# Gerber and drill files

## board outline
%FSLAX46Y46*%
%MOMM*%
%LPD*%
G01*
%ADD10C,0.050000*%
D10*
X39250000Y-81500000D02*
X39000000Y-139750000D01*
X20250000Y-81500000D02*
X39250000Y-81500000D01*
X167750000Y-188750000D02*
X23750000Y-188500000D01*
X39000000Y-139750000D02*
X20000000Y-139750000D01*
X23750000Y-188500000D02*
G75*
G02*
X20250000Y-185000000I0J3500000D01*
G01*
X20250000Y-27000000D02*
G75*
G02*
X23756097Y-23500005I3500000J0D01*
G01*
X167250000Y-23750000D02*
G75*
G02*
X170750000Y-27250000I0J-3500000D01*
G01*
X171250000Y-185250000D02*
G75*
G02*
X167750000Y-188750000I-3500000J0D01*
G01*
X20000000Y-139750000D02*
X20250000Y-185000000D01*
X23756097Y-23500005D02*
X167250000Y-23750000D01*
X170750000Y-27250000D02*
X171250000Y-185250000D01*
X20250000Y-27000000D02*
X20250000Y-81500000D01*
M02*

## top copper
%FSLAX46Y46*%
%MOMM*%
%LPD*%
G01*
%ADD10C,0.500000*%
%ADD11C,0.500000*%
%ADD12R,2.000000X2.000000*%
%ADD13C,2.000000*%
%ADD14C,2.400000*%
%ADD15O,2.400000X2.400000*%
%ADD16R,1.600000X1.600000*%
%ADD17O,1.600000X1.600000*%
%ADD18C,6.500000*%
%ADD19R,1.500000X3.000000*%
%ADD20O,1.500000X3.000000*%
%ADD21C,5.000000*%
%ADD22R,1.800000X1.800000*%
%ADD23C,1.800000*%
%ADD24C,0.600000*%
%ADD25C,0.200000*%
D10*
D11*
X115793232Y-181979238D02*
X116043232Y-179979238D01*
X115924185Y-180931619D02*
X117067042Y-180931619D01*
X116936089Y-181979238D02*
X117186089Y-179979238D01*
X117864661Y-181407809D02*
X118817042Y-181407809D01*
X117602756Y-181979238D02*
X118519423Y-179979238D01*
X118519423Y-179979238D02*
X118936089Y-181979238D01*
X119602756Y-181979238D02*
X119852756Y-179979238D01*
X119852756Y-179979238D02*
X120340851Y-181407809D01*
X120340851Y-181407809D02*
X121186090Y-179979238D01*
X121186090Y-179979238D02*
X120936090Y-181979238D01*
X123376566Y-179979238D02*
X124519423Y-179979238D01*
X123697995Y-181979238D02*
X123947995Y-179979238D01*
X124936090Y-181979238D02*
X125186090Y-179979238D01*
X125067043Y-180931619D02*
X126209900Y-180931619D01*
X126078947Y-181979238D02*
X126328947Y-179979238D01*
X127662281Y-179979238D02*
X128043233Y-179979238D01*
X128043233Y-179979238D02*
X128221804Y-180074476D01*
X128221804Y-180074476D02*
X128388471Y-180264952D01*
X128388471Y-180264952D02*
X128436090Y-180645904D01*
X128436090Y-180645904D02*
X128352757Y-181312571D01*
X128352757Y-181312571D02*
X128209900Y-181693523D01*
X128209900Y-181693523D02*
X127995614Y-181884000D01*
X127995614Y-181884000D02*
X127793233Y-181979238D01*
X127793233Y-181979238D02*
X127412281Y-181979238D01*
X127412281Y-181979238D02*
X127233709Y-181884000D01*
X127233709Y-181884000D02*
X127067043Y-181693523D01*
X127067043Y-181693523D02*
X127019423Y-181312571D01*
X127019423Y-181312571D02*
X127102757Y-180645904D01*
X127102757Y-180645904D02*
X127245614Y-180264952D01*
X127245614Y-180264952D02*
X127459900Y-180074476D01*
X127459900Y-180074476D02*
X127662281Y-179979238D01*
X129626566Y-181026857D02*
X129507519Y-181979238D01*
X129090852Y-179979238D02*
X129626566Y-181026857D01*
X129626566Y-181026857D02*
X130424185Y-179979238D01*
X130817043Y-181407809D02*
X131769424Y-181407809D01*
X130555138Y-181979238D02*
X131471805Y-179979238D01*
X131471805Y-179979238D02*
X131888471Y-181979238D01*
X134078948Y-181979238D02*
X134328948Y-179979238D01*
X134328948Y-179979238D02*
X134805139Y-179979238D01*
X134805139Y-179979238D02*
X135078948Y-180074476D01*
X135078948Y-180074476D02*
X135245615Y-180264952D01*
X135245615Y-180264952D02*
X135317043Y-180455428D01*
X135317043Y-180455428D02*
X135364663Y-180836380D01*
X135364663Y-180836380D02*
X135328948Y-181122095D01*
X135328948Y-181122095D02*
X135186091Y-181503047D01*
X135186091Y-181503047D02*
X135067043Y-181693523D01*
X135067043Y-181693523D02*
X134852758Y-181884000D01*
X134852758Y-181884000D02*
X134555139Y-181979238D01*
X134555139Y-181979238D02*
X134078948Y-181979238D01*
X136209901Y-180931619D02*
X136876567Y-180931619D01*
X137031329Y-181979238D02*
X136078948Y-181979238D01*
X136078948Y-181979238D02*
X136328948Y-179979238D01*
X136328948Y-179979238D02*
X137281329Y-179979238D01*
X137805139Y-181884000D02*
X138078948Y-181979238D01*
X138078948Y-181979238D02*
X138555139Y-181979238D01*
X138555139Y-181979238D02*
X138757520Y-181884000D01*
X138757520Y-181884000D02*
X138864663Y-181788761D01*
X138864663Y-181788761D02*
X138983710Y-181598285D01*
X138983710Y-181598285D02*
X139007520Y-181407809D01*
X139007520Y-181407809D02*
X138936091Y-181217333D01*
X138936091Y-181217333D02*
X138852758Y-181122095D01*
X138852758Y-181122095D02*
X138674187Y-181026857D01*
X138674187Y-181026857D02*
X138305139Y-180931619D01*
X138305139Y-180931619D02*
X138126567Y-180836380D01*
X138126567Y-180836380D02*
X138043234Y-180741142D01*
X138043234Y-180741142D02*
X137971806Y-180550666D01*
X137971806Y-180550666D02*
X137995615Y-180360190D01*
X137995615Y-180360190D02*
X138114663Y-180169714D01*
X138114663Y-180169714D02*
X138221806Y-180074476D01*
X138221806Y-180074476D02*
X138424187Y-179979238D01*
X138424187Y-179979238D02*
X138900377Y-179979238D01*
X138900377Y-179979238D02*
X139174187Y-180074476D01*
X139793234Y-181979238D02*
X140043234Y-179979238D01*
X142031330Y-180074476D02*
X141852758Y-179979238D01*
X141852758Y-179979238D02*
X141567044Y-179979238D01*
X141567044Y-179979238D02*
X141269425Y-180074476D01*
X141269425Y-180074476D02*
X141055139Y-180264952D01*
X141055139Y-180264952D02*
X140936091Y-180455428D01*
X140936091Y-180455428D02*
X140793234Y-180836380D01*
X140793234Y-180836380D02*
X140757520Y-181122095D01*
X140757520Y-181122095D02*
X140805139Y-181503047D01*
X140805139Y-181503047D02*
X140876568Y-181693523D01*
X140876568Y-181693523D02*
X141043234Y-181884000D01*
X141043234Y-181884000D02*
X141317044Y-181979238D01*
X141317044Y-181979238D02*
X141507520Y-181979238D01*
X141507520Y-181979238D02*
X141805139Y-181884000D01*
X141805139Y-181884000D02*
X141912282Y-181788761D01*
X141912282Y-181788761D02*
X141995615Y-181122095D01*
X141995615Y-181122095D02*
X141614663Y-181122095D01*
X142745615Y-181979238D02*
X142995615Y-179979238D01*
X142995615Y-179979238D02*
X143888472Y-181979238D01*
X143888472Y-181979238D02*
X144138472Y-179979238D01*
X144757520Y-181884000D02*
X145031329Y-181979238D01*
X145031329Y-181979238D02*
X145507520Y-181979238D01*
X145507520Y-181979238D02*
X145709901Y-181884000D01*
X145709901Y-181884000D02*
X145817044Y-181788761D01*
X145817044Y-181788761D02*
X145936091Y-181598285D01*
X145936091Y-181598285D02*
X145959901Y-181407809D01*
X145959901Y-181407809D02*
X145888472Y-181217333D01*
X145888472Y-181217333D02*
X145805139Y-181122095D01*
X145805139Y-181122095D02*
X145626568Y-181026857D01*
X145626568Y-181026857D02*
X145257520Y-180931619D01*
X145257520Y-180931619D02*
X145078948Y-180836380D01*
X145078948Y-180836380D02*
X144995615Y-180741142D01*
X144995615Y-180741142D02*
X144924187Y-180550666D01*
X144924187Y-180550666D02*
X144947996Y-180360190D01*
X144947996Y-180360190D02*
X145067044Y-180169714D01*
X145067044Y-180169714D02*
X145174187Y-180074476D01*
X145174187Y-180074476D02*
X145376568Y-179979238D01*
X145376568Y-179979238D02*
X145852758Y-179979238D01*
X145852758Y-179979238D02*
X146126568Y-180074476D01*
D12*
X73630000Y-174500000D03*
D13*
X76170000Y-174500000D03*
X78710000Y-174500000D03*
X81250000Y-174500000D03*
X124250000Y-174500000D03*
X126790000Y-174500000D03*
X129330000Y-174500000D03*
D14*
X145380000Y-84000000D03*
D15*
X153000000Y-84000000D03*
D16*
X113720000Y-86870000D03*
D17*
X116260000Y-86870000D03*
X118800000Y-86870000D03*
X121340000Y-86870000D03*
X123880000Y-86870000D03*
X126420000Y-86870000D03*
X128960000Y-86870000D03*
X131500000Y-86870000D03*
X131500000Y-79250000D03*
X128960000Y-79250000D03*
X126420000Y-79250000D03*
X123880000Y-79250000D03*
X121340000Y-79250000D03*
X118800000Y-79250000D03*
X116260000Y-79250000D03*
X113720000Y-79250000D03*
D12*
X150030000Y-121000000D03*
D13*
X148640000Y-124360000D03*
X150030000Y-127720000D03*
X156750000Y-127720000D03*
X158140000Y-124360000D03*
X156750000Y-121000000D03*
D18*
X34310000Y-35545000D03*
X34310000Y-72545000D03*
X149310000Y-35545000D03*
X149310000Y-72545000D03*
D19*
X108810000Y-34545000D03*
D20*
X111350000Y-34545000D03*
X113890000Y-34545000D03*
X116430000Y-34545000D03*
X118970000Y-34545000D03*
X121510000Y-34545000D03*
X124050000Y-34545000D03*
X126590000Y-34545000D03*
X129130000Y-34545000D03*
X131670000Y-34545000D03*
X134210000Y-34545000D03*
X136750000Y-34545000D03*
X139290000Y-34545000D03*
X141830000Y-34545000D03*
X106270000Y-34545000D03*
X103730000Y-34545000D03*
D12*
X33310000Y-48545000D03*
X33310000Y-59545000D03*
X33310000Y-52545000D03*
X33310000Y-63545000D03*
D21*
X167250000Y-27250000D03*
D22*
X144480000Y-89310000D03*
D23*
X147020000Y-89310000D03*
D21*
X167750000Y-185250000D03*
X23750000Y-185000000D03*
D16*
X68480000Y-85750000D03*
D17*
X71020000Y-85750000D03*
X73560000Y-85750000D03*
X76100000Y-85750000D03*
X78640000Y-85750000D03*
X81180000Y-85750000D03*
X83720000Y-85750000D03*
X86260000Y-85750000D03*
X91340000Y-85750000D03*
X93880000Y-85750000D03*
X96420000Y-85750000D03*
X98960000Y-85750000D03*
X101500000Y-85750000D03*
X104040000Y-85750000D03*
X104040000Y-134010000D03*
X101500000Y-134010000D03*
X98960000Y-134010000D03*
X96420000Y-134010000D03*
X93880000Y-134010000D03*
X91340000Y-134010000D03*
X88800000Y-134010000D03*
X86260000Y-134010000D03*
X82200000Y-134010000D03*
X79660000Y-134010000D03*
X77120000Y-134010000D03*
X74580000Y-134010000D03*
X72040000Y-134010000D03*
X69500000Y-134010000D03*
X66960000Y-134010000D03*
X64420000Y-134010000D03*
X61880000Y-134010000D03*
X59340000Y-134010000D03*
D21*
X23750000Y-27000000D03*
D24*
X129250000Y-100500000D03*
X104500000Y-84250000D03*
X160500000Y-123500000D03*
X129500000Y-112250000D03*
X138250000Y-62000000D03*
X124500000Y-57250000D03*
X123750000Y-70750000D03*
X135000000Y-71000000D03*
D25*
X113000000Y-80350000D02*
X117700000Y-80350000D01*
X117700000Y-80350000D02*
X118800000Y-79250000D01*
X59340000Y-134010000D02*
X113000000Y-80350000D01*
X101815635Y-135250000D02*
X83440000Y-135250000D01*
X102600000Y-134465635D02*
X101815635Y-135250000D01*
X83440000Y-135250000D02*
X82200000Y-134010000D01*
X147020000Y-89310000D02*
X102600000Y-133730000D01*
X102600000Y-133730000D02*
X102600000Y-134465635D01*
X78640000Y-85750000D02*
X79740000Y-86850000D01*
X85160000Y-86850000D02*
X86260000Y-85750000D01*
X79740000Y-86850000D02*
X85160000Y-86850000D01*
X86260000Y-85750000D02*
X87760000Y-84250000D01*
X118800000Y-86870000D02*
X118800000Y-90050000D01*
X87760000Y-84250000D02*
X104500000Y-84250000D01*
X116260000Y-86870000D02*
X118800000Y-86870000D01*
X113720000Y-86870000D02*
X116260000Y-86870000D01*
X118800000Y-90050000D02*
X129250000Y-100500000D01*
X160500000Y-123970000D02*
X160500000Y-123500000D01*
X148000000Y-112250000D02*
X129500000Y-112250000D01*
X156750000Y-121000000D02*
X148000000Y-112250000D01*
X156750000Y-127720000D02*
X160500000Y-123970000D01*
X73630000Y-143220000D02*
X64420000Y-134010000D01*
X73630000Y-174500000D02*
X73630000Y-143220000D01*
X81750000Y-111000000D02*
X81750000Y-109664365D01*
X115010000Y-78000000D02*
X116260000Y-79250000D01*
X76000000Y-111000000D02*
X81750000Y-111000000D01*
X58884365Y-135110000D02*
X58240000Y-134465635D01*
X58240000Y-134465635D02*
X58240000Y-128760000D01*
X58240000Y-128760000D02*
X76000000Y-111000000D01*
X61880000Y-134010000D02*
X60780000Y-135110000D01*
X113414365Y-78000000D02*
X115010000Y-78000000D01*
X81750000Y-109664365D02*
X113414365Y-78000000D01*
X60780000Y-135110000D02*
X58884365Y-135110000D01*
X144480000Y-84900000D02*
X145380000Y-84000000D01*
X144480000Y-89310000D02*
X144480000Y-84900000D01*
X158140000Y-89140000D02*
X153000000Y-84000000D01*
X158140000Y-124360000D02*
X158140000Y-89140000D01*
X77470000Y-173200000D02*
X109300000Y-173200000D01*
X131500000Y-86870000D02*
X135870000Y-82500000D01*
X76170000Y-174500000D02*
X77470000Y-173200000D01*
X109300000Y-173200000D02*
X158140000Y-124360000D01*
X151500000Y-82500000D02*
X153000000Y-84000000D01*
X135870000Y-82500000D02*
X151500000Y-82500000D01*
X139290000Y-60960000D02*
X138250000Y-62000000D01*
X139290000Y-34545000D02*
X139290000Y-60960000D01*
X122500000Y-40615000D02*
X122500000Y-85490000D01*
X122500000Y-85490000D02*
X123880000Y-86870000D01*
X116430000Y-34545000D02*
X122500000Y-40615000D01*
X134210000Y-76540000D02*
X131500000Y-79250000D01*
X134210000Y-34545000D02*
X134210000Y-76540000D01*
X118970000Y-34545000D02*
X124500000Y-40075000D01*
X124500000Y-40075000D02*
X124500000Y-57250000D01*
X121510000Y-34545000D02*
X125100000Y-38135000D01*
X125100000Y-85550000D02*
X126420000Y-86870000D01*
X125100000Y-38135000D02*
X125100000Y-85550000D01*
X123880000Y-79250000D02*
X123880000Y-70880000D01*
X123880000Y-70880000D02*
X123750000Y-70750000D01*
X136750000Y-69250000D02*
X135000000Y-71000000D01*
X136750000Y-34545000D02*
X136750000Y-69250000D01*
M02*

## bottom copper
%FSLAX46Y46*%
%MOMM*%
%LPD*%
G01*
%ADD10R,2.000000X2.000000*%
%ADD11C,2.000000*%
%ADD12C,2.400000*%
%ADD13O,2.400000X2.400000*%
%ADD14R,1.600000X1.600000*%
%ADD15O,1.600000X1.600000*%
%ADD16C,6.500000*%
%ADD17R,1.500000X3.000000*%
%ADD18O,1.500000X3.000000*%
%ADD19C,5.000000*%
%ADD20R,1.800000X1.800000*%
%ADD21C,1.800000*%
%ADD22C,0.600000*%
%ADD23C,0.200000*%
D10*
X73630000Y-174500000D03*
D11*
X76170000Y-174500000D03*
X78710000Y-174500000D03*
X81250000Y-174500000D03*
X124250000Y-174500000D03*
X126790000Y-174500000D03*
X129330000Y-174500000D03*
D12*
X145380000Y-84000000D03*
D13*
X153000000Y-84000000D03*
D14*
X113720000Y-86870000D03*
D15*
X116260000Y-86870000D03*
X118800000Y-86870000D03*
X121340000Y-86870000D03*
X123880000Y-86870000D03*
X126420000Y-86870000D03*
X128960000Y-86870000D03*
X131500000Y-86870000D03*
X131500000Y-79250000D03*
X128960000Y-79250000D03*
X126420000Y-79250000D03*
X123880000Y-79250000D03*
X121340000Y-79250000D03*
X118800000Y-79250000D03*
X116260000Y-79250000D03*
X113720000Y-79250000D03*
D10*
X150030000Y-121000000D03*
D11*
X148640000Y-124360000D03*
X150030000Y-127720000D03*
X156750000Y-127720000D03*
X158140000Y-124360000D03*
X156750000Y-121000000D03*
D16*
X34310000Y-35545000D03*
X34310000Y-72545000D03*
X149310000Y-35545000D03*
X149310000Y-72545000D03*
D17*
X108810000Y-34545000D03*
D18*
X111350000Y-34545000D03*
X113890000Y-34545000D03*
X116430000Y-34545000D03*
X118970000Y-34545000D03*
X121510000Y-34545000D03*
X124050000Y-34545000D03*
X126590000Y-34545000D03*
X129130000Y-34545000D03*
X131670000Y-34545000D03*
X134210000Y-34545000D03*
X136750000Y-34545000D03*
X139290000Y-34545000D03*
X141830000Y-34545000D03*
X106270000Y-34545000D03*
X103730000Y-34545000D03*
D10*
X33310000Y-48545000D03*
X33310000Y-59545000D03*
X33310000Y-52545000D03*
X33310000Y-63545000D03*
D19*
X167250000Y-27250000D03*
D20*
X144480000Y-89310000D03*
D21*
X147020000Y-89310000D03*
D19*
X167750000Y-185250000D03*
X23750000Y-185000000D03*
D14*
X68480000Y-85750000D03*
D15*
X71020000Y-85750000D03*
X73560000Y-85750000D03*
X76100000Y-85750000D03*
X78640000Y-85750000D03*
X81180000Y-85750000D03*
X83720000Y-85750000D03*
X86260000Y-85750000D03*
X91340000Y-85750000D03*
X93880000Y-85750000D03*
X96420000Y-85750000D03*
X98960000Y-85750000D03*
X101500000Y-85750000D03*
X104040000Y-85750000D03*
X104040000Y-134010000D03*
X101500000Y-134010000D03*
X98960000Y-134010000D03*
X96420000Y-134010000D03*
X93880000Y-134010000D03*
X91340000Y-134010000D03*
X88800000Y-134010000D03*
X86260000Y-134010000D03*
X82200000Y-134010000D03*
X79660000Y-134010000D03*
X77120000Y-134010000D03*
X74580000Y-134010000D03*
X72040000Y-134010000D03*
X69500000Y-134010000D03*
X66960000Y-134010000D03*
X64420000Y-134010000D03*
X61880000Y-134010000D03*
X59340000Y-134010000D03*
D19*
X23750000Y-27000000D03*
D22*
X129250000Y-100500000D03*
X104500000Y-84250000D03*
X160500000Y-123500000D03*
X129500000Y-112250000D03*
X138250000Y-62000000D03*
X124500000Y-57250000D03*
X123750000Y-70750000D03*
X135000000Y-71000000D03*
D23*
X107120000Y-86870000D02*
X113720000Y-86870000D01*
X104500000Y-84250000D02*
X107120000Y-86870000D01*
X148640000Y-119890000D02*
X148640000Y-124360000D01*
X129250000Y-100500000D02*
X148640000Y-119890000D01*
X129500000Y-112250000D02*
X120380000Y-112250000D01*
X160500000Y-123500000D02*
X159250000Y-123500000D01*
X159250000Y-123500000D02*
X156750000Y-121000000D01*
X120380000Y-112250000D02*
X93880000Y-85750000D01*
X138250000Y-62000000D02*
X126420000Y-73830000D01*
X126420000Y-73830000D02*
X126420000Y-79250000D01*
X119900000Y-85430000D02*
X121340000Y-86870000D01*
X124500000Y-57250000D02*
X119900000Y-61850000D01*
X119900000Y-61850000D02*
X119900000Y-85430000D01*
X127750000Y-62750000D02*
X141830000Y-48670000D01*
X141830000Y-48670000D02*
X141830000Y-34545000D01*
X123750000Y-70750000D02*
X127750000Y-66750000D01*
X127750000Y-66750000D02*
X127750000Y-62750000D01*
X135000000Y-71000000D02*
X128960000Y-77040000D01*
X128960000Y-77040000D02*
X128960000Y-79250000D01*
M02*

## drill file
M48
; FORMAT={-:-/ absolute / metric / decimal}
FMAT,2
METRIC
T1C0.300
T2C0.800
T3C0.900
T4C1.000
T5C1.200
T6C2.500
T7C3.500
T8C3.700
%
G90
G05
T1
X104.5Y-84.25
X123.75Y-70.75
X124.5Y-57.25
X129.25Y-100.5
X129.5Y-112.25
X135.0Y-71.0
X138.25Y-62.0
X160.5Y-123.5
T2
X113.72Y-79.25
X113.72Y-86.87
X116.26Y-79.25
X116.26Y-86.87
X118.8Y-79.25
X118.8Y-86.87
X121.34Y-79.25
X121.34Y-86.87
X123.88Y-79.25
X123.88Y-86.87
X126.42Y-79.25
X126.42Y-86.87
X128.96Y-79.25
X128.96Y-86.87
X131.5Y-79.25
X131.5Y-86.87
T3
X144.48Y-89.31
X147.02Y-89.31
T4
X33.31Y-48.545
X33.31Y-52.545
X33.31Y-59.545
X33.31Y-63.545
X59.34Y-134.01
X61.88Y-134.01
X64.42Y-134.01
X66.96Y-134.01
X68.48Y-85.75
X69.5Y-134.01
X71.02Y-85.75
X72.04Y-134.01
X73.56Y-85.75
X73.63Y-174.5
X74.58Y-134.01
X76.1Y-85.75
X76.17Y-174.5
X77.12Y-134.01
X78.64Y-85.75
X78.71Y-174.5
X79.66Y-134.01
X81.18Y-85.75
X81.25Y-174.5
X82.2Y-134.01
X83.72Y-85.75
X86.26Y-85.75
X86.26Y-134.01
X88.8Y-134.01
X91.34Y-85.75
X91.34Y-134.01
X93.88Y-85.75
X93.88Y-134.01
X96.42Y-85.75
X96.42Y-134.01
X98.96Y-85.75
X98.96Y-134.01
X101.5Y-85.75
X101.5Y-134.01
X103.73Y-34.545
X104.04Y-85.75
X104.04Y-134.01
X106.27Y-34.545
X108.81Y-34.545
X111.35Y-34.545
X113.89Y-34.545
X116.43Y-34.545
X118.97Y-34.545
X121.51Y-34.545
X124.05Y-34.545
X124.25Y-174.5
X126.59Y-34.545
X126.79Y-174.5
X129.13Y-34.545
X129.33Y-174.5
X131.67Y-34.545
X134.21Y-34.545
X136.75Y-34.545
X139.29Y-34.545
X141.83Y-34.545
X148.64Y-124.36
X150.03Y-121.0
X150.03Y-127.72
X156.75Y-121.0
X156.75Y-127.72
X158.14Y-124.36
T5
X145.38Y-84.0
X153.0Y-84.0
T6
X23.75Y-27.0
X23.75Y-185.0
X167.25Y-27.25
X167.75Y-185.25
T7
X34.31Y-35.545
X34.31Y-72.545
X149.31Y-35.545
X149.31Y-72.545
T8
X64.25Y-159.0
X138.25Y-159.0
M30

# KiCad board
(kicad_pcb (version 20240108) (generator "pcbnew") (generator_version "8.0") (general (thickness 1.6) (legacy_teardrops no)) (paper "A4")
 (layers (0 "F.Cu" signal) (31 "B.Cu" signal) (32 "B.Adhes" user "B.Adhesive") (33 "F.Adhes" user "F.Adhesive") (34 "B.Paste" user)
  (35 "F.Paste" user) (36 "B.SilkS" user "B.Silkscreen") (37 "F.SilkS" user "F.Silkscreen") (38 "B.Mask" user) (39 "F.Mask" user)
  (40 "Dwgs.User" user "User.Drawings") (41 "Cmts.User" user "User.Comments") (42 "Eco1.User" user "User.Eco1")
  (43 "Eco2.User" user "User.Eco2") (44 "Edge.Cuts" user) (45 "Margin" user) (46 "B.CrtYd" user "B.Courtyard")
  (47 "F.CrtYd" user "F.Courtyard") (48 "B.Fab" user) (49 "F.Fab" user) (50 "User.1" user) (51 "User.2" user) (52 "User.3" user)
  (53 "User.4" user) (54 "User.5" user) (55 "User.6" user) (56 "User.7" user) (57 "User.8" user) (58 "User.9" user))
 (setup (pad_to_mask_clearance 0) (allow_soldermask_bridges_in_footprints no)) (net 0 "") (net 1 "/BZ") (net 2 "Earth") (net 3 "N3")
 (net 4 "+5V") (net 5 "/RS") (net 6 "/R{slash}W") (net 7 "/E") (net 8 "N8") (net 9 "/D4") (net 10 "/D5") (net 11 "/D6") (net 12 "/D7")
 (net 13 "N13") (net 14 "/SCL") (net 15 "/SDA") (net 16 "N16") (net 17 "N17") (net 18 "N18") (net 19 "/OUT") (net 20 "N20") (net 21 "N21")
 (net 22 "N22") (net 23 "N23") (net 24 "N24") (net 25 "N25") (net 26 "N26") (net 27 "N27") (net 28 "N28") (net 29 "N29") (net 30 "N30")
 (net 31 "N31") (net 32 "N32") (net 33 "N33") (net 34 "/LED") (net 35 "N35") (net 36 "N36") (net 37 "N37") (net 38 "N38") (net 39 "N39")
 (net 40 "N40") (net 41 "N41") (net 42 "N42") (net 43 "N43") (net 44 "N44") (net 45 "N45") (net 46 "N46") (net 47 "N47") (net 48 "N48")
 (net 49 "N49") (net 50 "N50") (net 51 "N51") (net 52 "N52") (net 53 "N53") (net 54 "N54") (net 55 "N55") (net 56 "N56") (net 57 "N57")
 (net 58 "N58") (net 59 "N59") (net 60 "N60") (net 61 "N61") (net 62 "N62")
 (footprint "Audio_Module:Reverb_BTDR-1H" (layer "F.Cu") (at 73.63 174.5)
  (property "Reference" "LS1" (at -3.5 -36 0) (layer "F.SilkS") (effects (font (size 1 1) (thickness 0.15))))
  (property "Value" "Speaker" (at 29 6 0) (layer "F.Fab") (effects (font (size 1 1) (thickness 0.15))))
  (pad "" np_thru_hole circle (at -9.38 -15.5) (size 3.7 3.7) (drill 3.7) (layers "*.Cu" "*.Mask"))
  (pad "" np_thru_hole circle (at 64.62 -15.5) (size 3.7 3.7) (drill 3.7) (layers "*.Cu" "*.Mask"))
  (pad "1" thru_hole rect (at 0 0) (size 2 2) (drill 1) (layers "*.Cu" "*.Mask") (remove_unused_layers no) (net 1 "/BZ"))
  (pad "2" thru_hole circle (at 2.54 0) (size 2 2) (drill 1) (layers "*.Cu" "*.Mask") (remove_unused_layers no) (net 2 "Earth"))
  (pad "3" thru_hole circle (at 5.08 0) (size 2 2) (drill 1) (layers "*.Cu" "*.Mask") (remove_unused_layers no))
  (pad "4" thru_hole circle (at 7.62 0) (size 2 2) (drill 1) (layers "*.Cu" "*.Mask") (remove_unused_layers no))
  (pad "5" thru_hole circle (at 50.62 0) (size 2 2) (drill 1) (layers "*.Cu" "*.Mask") (remove_unused_layers no))
  (pad "6" thru_hole circle (at 53.16 0) (size 2 2) (drill 1) (layers "*.Cu" "*.Mask") (remove_unused_layers no))
  (pad "7" thru_hole circle (at 55.7 0) (size 2 2) (drill 1) (layers "*.Cu" "*.Mask") (remove_unused_layers no)))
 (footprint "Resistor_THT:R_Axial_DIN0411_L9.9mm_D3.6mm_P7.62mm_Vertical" (layer "F.Cu") (at 145.38 84)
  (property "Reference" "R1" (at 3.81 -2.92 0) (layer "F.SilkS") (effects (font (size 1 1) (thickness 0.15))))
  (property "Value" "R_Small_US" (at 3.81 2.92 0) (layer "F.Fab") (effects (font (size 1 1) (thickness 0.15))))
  (pad "1" thru_hole circle (at 0 0) (size 2.4 2.4) (drill 1.2) (layers "*.Cu" "*.Mask") (remove_unused_layers no) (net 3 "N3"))
  (pad "2" thru_hole oval (at 7.62 0) (size 2.4 2.4) (drill 1.2) (layers "*.Cu" "*.Mask") (remove_unused_layers no) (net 2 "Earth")))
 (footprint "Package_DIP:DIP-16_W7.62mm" (layer "F.Cu") (at 113.72 86.87 90)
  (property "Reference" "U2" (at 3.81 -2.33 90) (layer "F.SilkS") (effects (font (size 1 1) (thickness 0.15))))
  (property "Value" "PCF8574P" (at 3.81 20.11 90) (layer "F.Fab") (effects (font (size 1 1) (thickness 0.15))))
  (pad "1" thru_hole rect (at 0 0 90) (size 1.6 1.6) (drill 0.8) (layers "*.Cu" "*.Mask") (remove_unused_layers no) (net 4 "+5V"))
  (pad "2" thru_hole oval (at 0 2.54 90) (size 1.6 1.6) (drill 0.8) (layers "*.Cu" "*.Mask") (remove_unused_layers no) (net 4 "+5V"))
  (pad "3" thru_hole oval (at 0 5.08 90) (size 1.6 1.6) (drill 0.8) (layers "*.Cu" "*.Mask") (remove_unused_layers no) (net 4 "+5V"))
  (pad "4" thru_hole oval (at 0 7.62 90) (size 1.6 1.6) (drill 0.8) (layers "*.Cu" "*.Mask") (remove_unused_layers no) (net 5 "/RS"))
  (pad "5" thru_hole oval (at 0 10.16 90) (size 1.6 1.6) (drill 0.8) (layers "*.Cu" "*.Mask") (remove_unused_layers no) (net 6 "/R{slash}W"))
  (pad "6" thru_hole oval (at 0 12.7 90) (size 1.6 1.6) (drill 0.8) (layers "*.Cu" "*.Mask") (remove_unused_layers no) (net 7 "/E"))
  (pad "7" thru_hole oval (at 0 15.24 90) (size 1.6 1.6) (drill 0.8) (layers "*.Cu" "*.Mask") (remove_unused_layers no) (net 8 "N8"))
  (pad "8" thru_hole oval (at 0 17.78 90) (size 1.6 1.6) (drill 0.8) (layers "*.Cu" "*.Mask") (remove_unused_layers no) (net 2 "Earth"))
  (pad "9" thru_hole oval (at 7.62 17.78 90) (size 1.6 1.6) (drill 0.8) (layers "*.Cu" "*.Mask") (remove_unused_layers no) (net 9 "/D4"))
  (pad "10" thru_hole oval (at 7.62 15.24 90) (size 1.6 1.6) (drill 0.8) (layers "*.Cu" "*.Mask") (remove_unused_layers no) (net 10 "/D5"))
  (pad "11" thru_hole oval (at 7.62 12.7 90) (size 1.6 1.6) (drill 0.8) (layers "*.Cu" "*.Mask") (remove_unused_layers no) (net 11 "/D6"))
  (pad "12" thru_hole oval (at 7.62 10.16 90) (size 1.6 1.6) (drill 0.8) (layers "*.Cu" "*.Mask") (remove_unused_layers no) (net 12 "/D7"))
  (pad "13" thru_hole oval (at 7.62 7.62 90) (size 1.6 1.6) (drill 0.8) (layers "*.Cu" "*.Mask") (remove_unused_layers no) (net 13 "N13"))
  (pad "14" thru_hole oval (at 7.62 5.08 90) (size 1.6 1.6) (drill 0.8) (layers "*.Cu" "*.Mask") (remove_unused_layers no) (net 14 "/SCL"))
  (pad "15" thru_hole oval (at 7.62 2.54 90) (size 1.6 1.6) (drill 0.8) (layers "*.Cu" "*.Mask") (remove_unused_layers no) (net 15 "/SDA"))
  (pad "16" thru_hole oval (at 7.62 0 90) (size 1.6 1.6) (drill 0.8) (layers "*.Cu" "*.Mask") (remove_unused_layers no) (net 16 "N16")))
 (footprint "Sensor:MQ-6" (layer "F.Cu") (at 150.03 121)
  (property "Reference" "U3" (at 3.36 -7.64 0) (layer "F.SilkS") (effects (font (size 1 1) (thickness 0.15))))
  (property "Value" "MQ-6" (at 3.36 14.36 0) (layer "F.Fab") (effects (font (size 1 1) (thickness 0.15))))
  (pad "1" thru_hole rect (at 0 0) (size 2 2) (drill 1) (layers "*.Cu" "*.Mask") (remove_unused_layers no) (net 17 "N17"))
  (pad "2" thru_hole circle (at -1.39 3.36) (size 2 2) (drill 1) (layers "*.Cu" "*.Mask") (remove_unused_layers no) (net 4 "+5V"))
  (pad "3" thru_hole circle (at 0 6.72 90) (size 2 2) (drill 1) (layers "*.Cu" "*.Mask") (remove_unused_layers no) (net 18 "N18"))
  (pad "4" thru_hole circle (at 6.72 6.72 180) (size 2 2) (drill 1) (layers "*.Cu" "*.Mask") (remove_unused_layers no) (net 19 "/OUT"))
  (pad "5" thru_hole circle (at 8.11 3.36) (size 2 2) (drill 1) (layers "*.Cu" "*.Mask") (remove_unused_layers no) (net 2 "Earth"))
  (pad "6" thru_hole circle (at 6.72 0 270) (size 2 2) (drill 1) (layers "*.Cu" "*.Mask") (remove_unused_layers no) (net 19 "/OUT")))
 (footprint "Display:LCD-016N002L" (layer "F.Cu") (at 108.81 34.545)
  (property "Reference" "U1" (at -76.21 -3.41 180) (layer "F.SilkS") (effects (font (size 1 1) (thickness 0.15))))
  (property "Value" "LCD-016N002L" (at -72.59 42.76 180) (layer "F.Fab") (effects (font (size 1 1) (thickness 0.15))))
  (pad "" thru_hole circle (at -74.5 1 180) (size 6.5 6.5) (drill 3.5) (layers "*.Cu" "*.Mask") (remove_unused_layers no))
  (pad "" thru_hole circle (at -74.5 38 180) (size 6.5 6.5) (drill 3.5) (layers "*.Cu" "*.Mask") (remove_unused_layers no))
  (pad "" thru_hole circle (at 40.5 1 180) (size 6.5 6.5) (drill 3.5) (layers "*.Cu" "*.Mask") (remove_unused_layers no))
  (pad "" thru_hole circle (at 40.5 38 180) (size 6.5 6.5) (drill 3.5) (layers "*.Cu" "*.Mask") (remove_unused_layers no))
  (pad "1" thru_hole rect (at 0 0 180) (size 1.5 3) (drill 1) (layers "*.Cu" "*.Mask") (remove_unused_layers no) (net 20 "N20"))
  (pad "2" thru_hole oval (at 2.54 0 180) (size 1.5 3) (drill 1) (layers "*.Cu" "*.Mask") (remove_unused_layers no) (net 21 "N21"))
  (pad "3" thru_hole oval (at 5.08 0 180) (size 1.5 3) (drill 1) (layers "*.Cu" "*.Mask") (remove_unused_layers no) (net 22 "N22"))
  (pad "4" thru_hole oval (at 7.62 0 180) (size 1.5 3) (drill 1) (layers "*.Cu" "*.Mask") (remove_unused_layers no) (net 6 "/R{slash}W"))
  (pad "5" thru_hole oval (at 10.16 0 180) (size 1.5 3) (drill 1) (layers "*.Cu" "*.Mask") (remove_unused_layers no) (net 5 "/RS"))
  (pad "6" thru_hole oval (at 12.7 0 180) (size 1.5 3) (drill 1) (layers "*.Cu" "*.Mask") (remove_unused_layers no) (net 7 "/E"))
  (pad "7" thru_hole oval (at 15.24 0 180) (size 1.5 3) (drill 1) (layers "*.Cu" "*.Mask") (remove_unused_layers no) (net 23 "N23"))
  (pad "8" thru_hole oval (at 17.78 0 180) (size 1.5 3) (drill 1) (layers "*.Cu" "*.Mask") (remove_unused_layers no) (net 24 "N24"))
  (pad "9" thru_hole oval (at 20.32 0 180) (size 1.5 3) (drill 1) (layers "*.Cu" "*.Mask") (remove_unused_layers no) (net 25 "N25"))
  (pad "10" thru_hole oval (at 22.86 0 180) (size 1.5 3) (drill 1) (layers "*.Cu" "*.Mask") (remove_unused_layers no) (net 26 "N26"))
  (pad "11" thru_hole oval (at 25.4 0 180) (size 1.5 3) (drill 1) (layers "*.Cu" "*.Mask") (remove_unused_layers no) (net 9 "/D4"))
  (pad "12" thru_hole oval (at 27.94 0 180) (size 1.5 3) (drill 1) (layers "*.Cu" "*.Mask") (remove_unused_layers no) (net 10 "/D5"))
  (pad "13" thru_hole oval (at 30.48 0 180) (size 1.5 3) (drill 1) (layers "*.Cu" "*.Mask") (remove_unused_layers no) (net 11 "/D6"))
  (pad "14" thru_hole oval (at 33.02 0 180) (size 1.5 3) (drill 1) (layers "*.Cu" "*.Mask") (remove_unused_layers no) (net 12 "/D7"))
  (pad "15" thru_hole oval (at -2.54 0 180) (size 1.5 3) (drill 1) (layers "*.Cu" "*.Mask") (remove_unused_layers no) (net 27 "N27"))
  (pad "16" thru_hole oval (at -5.08 0 180) (size 1.5 3) (drill 1) (layers "*.Cu" "*.Mask") (remove_unused_layers no) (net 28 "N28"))
  (pad "A1" thru_hole rect (at -75.5 14 180) (size 2 2) (drill 1) (layers "*.Cu" "*.Mask") (remove_unused_layers no) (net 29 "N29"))
  (pad "A2" thru_hole rect (at -75.5 25 180) (size 2 2) (drill 1) (layers "*.Cu" "*.Mask") (remove_unused_layers no) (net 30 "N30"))
  (pad "K1" thru_hole rect (at -75.5 18 180) (size 2 2) (drill 1) (layers "*.Cu" "*.Mask") (remove_unused_layers no) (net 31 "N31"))
  (pad "K2" thru_hole rect (at -75.5 29 180) (size 2 2) (drill 1) (layers "*.Cu" "*.Mask") (remove_unused_layers no) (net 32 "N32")))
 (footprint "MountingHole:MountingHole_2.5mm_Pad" (layer "F.Cu") (at 167.25 27.25)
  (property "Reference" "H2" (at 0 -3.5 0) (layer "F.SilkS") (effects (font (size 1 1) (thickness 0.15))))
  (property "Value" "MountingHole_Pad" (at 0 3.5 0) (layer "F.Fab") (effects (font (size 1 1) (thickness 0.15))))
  (pad "1" thru_hole circle (at 0 0) (size 5 5) (drill 2.5) (layers "*.Cu" "*.Mask") (remove_unused_layers no) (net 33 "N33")))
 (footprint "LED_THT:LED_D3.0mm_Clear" (layer "F.Cu") (at 144.48 89.31)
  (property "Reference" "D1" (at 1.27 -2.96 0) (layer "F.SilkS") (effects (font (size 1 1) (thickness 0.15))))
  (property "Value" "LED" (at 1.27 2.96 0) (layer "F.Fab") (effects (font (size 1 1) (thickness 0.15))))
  (pad "1" thru_hole rect (at 0 0) (size 1.8 1.8) (drill 0.9) (layers "*.Cu" "*.Mask") (remove_unused_layers no) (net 3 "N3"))
  (pad "2" thru_hole circle (at 2.54 0) (size 1.8 1.8) (drill 0.9) (layers "*.Cu" "*.Mask") (remove_unused_layers no) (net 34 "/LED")))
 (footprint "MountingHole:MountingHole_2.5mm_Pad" (layer "F.Cu") (at 167.75 185.25)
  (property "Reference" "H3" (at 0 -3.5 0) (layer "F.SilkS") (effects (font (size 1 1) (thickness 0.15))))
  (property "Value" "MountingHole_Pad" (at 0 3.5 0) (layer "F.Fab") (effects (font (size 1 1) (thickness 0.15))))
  (pad "1" thru_hole circle (at 0 0) (size 5 5) (drill 2.5) (layers "*.Cu" "*.Mask") (remove_unused_layers no) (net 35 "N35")))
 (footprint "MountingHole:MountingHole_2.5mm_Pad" (layer "F.Cu") (at 23.75 185)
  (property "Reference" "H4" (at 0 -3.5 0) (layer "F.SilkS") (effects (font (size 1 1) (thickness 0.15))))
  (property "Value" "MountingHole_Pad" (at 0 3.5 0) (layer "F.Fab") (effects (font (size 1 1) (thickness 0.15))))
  (pad "1" thru_hole circle (at 0 0) (size 5 5) (drill 2.5) (layers "*.Cu" "*.Mask") (remove_unused_layers no) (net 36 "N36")))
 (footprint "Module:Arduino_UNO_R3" (layer "F.Cu") (at 68.48 85.75)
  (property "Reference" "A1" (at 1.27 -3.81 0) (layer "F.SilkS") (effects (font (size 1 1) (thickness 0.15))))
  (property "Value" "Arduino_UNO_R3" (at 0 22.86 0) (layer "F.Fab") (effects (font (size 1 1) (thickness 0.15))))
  (pad "1" thru_hole rect (at 0 0 90) (size 1.6 1.6) (drill 1) (layers "*.Cu" "*.Mask") (remove_unused_layers no) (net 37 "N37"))
  (pad "2" thru_hole oval (at 2.54 0 90) (size 1.6 1.6) (drill 1) (layers "*.Cu" "*.Mask") (remove_unused_layers no) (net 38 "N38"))
  (pad "3" thru_hole oval (at 5.08 0 90) (size 1.6 1.6) (drill 1) (layers "*.Cu" "*.Mask") (remove_unused_layers no) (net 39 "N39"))
  (pad "4" thru_hole oval (at 7.62 0 90) (size 1.6 1.6) (drill 1) (layers "*.Cu" "*.Mask") (remove_unused_layers no) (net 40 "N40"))
  (pad "5" thru_hole oval (at 10.16 0 90) (size 1.6 1.6) (drill 1) (layers "*.Cu" "*.Mask") (remove_unused_layers no) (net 4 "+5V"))
  (pad "6" thru_hole oval (at 12.7 0 90) (size 1.6 1.6) (drill 1) (layers "*.Cu" "*.Mask") (remove_unused_layers no) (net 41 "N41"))
  (pad "7" thru_hole oval (at 15.24 0 90) (size 1.6 1.6) (drill 1) (layers "*.Cu" "*.Mask") (remove_unused_layers no) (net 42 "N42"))
  (pad "8" thru_hole oval (at 17.78 0 90) (size 1.6 1.6) (drill 1) (layers "*.Cu" "*.Mask") (remove_unused_layers no) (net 4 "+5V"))
  (pad "9" thru_hole oval (at 22.86 0 90) (size 1.6 1.6) (drill 1) (layers "*.Cu" "*.Mask") (remove_unused_layers no) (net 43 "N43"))
  (pad "10" thru_hole oval (at 25.4 0 90) (size 1.6 1.6) (drill 1) (layers "*.Cu" "*.Mask") (remove_unused_layers no) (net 19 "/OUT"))
  (pad "11" thru_hole oval (at 27.94 0 90) (size 1.6 1.6) (drill 1) (layers "*.Cu" "*.Mask") (remove_unused_layers no) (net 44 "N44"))
  (pad "12" thru_hole oval (at 30.48 0 90) (size 1.6 1.6) (drill 1) (layers "*.Cu" "*.Mask") (remove_unused_layers no) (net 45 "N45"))
  (pad "13" thru_hole oval (at 33.02 0 90) (size 1.6 1.6) (drill 1) (layers "*.Cu" "*.Mask") (remove_unused_layers no) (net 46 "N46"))
  (pad "14" thru_hole oval (at 35.56 0 90) (size 1.6 1.6) (drill 1) (layers "*.Cu" "*.Mask") (remove_unused_layers no) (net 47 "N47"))
  (pad "15" thru_hole oval (at 35.56 48.26 90) (size 1.6 1.6) (drill 1) (layers "*.Cu" "*.Mask") (remove_unused_layers no) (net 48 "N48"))
  (pad "16" thru_hole oval (at 33.02 48.26 90) (size 1.6 1.6) (drill 1) (layers "*.Cu" "*.Mask") (remove_unused_layers no) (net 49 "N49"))
  (pad "17" thru_hole oval (at 30.48 48.26 90) (size 1.6 1.6) (drill 1) (layers "*.Cu" "*.Mask") (remove_unused_layers no) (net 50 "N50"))
  (pad "18" thru_hole oval (at 27.94 48.26 90) (size 1.6 1.6) (drill 1) (layers "*.Cu" "*.Mask") (remove_unused_layers no) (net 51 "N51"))
  (pad "19" thru_hole oval (at 25.4 48.26 90) (size 1.6 1.6) (drill 1) (layers "*.Cu" "*.Mask") (remove_unused_layers no) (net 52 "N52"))
  (pad "20" thru_hole oval (at 22.86 48.26 90) (size 1.6 1.6) (drill 1) (layers "*.Cu" "*.Mask") (remove_unused_layers no) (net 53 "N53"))
  (pad "21" thru_hole oval (at 20.32 48.26 90) (size 1.6 1.6) (drill 1) (layers "*.Cu" "*.Mask") (remove_unused_layers no) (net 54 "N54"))
  (pad "22" thru_hole oval (at 17.78 48.26 90) (size 1.6 1.6) (drill 1) (layers "*.Cu" "*.Mask") (remove_unused_layers no) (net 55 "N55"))
  (pad "23" thru_hole oval (at 13.72 48.26 90) (size 1.6 1.6) (drill 1) (layers "*.Cu" "*.Mask") (remove_unused_layers no) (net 34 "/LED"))
  (pad "24" thru_hole oval (at 11.18 48.26 90) (size 1.6 1.6) (drill 1) (layers "*.Cu" "*.Mask") (remove_unused_layers no) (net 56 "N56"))
  (pad "25" thru_hole oval (at 8.64 48.26 90) (size 1.6 1.6) (drill 1) (layers "*.Cu" "*.Mask") (remove_unused_layers no) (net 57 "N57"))
  (pad "26" thru_hole oval (at 6.1 48.26 90) (size 1.6 1.6) (drill 1) (layers "*.Cu" "*.Mask") (remove_unused_layers no) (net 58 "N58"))
  (pad "27" thru_hole oval (at 3.56 48.26 90) (size 1.6 1.6) (drill 1) (layers "*.Cu" "*.Mask") (remove_unused_layers no) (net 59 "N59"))
  (pad "28" thru_hole oval (at 1.02 48.26 90) (size 1.6 1.6) (drill 1) (layers "*.Cu" "*.Mask") (remove_unused_layers no) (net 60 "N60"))
  (pad "29" thru_hole oval (at -1.52 48.26 90) (size 1.6 1.6) (drill 1) (layers "*.Cu" "*.Mask") (remove_unused_layers no) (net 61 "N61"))
  (pad "30" thru_hole oval (at -4.06 48.26 90) (size 1.6 1.6) (drill 1) (layers "*.Cu" "*.Mask") (remove_unused_layers no) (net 1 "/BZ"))
  (pad "31" thru_hole oval (at -6.6 48.26 90) (size 1.6 1.6) (drill 1) (layers "*.Cu" "*.Mask") (remove_unused_layers no) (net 15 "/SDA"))
  (pad "32" thru_hole oval (at -9.14 48.26 90) (size 1.6 1.6) (drill 1) (layers "*.Cu" "*.Mask") (remove_unused_layers no) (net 14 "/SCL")))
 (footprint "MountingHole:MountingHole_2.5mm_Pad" (layer "F.Cu") (at 23.75 27)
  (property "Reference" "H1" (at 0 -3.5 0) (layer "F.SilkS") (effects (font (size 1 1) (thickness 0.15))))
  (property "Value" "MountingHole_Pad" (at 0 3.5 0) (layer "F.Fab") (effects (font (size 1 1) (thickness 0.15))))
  (pad "1" thru_hole circle (at 0 0) (size 5 5) (drill 2.5) (layers "*.Cu" "*.Mask") (remove_unused_layers no) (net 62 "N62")))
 (gr_line (start 39.25 81.5) (end 39 139.75) (stroke (width 0.05) (type default)) (layer "Edge.Cuts"))
 (gr_line (start 20.25 81.5) (end 39.25 81.5) (stroke (width 0.05) (type default)) (layer "Edge.Cuts"))
 (gr_line (start 167.75 188.75) (end 23.75 188.5) (stroke (width 0.05) (type default)) (layer "Edge.Cuts"))
 (gr_line (start 39 139.75) (end 20 139.75) (stroke (width 0.05) (type default)) (layer "Edge.Cuts"))
 (gr_arc (start 23.75 188.5) (mid 21.275126 187.474874) (end 20.25 185) (stroke (width 0.05) (type default)) (layer "Edge.Cuts"))
 (gr_arc (start 20.25 27) (mid 21.277283 24.522972) (end 23.756097 23.500005) (stroke (width 0.05) (type default)) (layer "Edge.Cuts"))
 (gr_arc (start 167.25 23.75) (mid 169.724874 24.775126) (end 170.75 27.25) (stroke (width 0.05) (type default)) (layer "Edge.Cuts"))
 (gr_arc (start 171.25 185.25) (mid 170.224874 187.724874) (end 167.75 188.75) (stroke (width 0.05) (type default)) (layer "Edge.Cuts"))
 (gr_line (start 20 139.75) (end 20.25 185) (stroke (width 0.05) (type default)) (layer "Edge.Cuts"))
 (gr_line (start 23.756097 23.500005) (end 167.25 23.75) (stroke (width 0.05) (type default)) (layer "Edge.Cuts"))
 (gr_line (start 170.75 27.25) (end 171.25 185.25) (stroke (width 0.05) (type default)) (layer "Edge.Cuts"))
 (gr_line (start 20.25 27) (end 20.25 81.5) (stroke (width 0.05) (type default)) (layer "Edge.Cuts"))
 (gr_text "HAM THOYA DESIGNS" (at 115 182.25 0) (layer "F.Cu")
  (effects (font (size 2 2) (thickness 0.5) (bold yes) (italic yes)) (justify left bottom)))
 (segment (start 113 80.35) (end 117.7 80.35) (width 0.2) (layer "F.Cu") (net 14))
 (segment (start 117.7 80.35) (end 118.8 79.25) (width 0.2) (layer "F.Cu") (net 14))
 (segment (start 59.34 134.01) (end 113 80.35) (width 0.2) (layer "F.Cu") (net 14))
 (segment (start 101.815635 135.25) (end 83.44 135.25) (width 0.2) (layer "F.Cu") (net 34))
 (segment (start 102.6 134.465635) (end 101.815635 135.25) (width 0.2) (layer "F.Cu") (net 34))
 (segment (start 83.44 135.25) (end 82.2 134.01) (width 0.2) (layer "F.Cu") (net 34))
 (segment (start 147.02 89.31) (end 102.6 133.73) (width 0.2) (layer "F.Cu") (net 34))
 (segment (start 102.6 133.73) (end 102.6 134.465635) (width 0.2) (layer "F.Cu") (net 34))
 (segment (start 78.64 85.75) (end 79.74 86.85) (width 0.2) (layer "F.Cu") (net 4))
 (segment (start 85.16 86.85) (end 86.26 85.75) (width 0.2) (layer "F.Cu") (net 4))
 (segment (start 79.74 86.85) (end 85.16 86.85) (width 0.2) (layer "F.Cu") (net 4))
 (segment (start 86.26 85.75) (end 87.76 84.25) (width 0.2) (layer "F.Cu") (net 4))
 (segment (start 118.8 86.87) (end 118.8 90.05) (width 0.2) (layer "F.Cu") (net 4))
 (segment (start 87.76 84.25) (end 104.5 84.25) (width 0.2) (layer "F.Cu") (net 4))
 (segment (start 116.26 86.87) (end 118.8 86.87) (width 0.2) (layer "F.Cu") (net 4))
 (segment (start 113.72 86.87) (end 116.26 86.87) (width 0.2) (layer "F.Cu") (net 4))
 (segment (start 118.8 90.05) (end 129.25 100.5) (width 0.2) (layer "F.Cu") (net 4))
 (via (at 129.25 100.5) (size 0.6) (drill 0.3) (layers "F.Cu" "B.Cu") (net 4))
 (via (at 104.5 84.25) (size 0.6) (drill 0.3) (layers "F.Cu" "B.Cu") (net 4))
 (segment (start 107.12 86.87) (end 113.72 86.87) (width 0.2) (layer "B.Cu") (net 4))
 (segment (start 104.5 84.25) (end 107.12 86.87) (width 0.2) (layer "B.Cu") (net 4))
 (segment (start 148.64 119.89) (end 148.64 124.36) (width 0.2) (layer "B.Cu") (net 4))
 (segment (start 129.25 100.5) (end 148.64 119.89) (width 0.2) (layer "B.Cu") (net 4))
 (segment (start 160.5 123.97) (end 160.5 123.5) (width 0.2) (layer "F.Cu") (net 19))
 (segment (start 148 112.25) (end 129.5 112.25) (width 0.2) (layer "F.Cu") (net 19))
 (segment (start 156.75 121) (end 148 112.25) (width 0.2) (layer "F.Cu") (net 19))
 (segment (start 156.75 127.72) (end 160.5 123.97) (width 0.2) (layer "F.Cu") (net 19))
 (via (at 160.5 123.5) (size 0.6) (drill 0.3) (layers "F.Cu" "B.Cu") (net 19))
 (via (at 129.5 112.25) (size 0.6) (drill 0.3) (layers "F.Cu" "B.Cu") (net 19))
 (segment (start 129.5 112.25) (end 120.38 112.25) (width 0.2) (layer "B.Cu") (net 19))
 (segment (start 160.5 123.5) (end 159.25 123.5) (width 0.2) (layer "B.Cu") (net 19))
 (segment (start 159.25 123.5) (end 156.75 121) (width 0.2) (layer "B.Cu") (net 19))
 (segment (start 120.38 112.25) (end 93.88 85.75) (width 0.2) (layer "B.Cu") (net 19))
 (segment (start 73.63 143.22) (end 64.42 134.01) (width 0.2) (layer "F.Cu") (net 1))
 (segment (start 73.63 174.5) (end 73.63 143.22) (width 0.2) (layer "F.Cu") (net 1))
 (segment (start 81.75 111) (end 81.75 109.664365) (width 0.2) (layer "F.Cu") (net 15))
 (segment (start 115.01 78) (end 116.26 79.25) (width 0.2) (layer "F.Cu") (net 15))
 (segment (start 76 111) (end 81.75 111) (width 0.2) (layer "F.Cu") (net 15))
 (segment (start 58.884365 135.11) (end 58.24 134.465635) (width 0.2) (layer "F.Cu") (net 15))
 (segment (start 58.24 134.465635) (end 58.24 128.76) (width 0.2) (layer "F.Cu") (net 15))
 (segment (start 58.24 128.76) (end 76 111) (width 0.2) (layer "F.Cu") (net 15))
 (segment (start 61.88 134.01) (end 60.78 135.11) (width 0.2) (layer "F.Cu") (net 15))
 (segment (start 113.414365 78) (end 115.01 78) (width 0.2) (layer "F.Cu") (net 15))
 (segment (start 81.75 109.664365) (end 113.414365 78) (width 0.2) (layer "F.Cu") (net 15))
 (segment (start 60.78 135.11) (end 58.884365 135.11) (width 0.2) (layer "F.Cu") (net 15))
 (segment (start 144.48 84.9) (end 145.38 84) (width 0.2) (layer "F.Cu") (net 3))
 (segment (start 144.48 89.31) (end 144.48 84.9) (width 0.2) (layer "F.Cu") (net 3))
 (segment (start 158.14 89.14) (end 153 84) (width 0.2) (layer "F.Cu") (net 2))
 (segment (start 158.14 124.36) (end 158.14 89.14) (width 0.2) (layer "F.Cu") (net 2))
 (segment (start 77.47 173.2) (end 109.3 173.2) (width 0.2) (layer "F.Cu") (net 2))
 (segment (start 131.5 86.87) (end 135.87 82.5) (width 0.2) (layer "F.Cu") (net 2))
 (segment (start 76.17 174.5) (end 77.47 173.2) (width 0.2) (layer "F.Cu") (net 2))
 (segment (start 109.3 173.2) (end 158.14 124.36) (width 0.2) (layer "F.Cu") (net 2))
 (segment (start 151.5 82.5) (end 153 84) (width 0.2) (layer "F.Cu") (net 2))
 (segment (start 135.87 82.5) (end 151.5 82.5) (width 0.2) (layer "F.Cu") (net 2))
 (segment (start 139.29 60.96) (end 138.25 62) (width 0.2) (layer "F.Cu") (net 11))
 (segment (start 139.29 34.545) (end 139.29 60.96) (width 0.2) (layer "F.Cu") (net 11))
 (via (at 138.25 62) (size 0.6) (drill 0.3) (layers "F.Cu" "B.Cu") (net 11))
 (segment (start 138.25 62) (end 126.42 73.83) (width 0.2) (layer "B.Cu") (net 11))
 (segment (start 126.42 73.83) (end 126.42 79.25) (width 0.2) (layer "B.Cu") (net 11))
 (segment (start 122.5 40.615) (end 122.5 85.49) (width 0.2) (layer "F.Cu") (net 6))
 (segment (start 122.5 85.49) (end 123.88 86.87) (width 0.2) (layer "F.Cu") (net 6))
 (segment (start 116.43 34.545) (end 122.5 40.615) (width 0.2) (layer "F.Cu") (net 6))
 (segment (start 134.21 76.54) (end 131.5 79.25) (width 0.2) (layer "F.Cu") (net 9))
 (segment (start 134.21 34.545) (end 134.21 76.54) (width 0.2) (layer "F.Cu") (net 9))
 (segment (start 118.97 34.545) (end 124.5 40.075) (width 0.2) (layer "F.Cu") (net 5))
 (segment (start 124.5 40.075) (end 124.5 57.25) (width 0.2) (layer "F.Cu") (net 5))
 (via (at 124.5 57.25) (size 0.6) (drill 0.3) (layers "F.Cu" "B.Cu") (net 5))
 (segment (start 119.9 85.43) (end 121.34 86.87) (width 0.2) (layer "B.Cu") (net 5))
 (segment (start 124.5 57.25) (end 119.9 61.85) (width 0.2) (layer "B.Cu") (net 5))
 (segment (start 119.9 61.85) (end 119.9 85.43) (width 0.2) (layer "B.Cu") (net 5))
 (segment (start 121.51 34.545) (end 125.1 38.135) (width 0.2) (layer "F.Cu") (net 7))
 (segment (start 125.1 85.55) (end 126.42 86.87) (width 0.2) (layer "F.Cu") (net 7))
 (segment (start 125.1 38.135) (end 125.1 85.55) (width 0.2) (layer "F.Cu") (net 7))
 (segment (start 123.88 79.25) (end 123.88 70.88) (width 0.2) (layer "F.Cu") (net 12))
 (segment (start 123.88 70.88) (end 123.75 70.75) (width 0.2) (layer "F.Cu") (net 12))
 (via (at 123.75 70.75) (size 0.6) (drill 0.3) (layers "F.Cu" "B.Cu") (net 12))
 (segment (start 127.75 62.75) (end 141.83 48.67) (width 0.2) (layer "B.Cu") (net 12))
 (segment (start 141.83 48.67) (end 141.83 34.545) (width 0.2) (layer "B.Cu") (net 12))
 (segment (start 123.75 70.75) (end 127.75 66.75) (width 0.2) (layer "B.Cu") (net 12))
 (segment (start 127.75 66.75) (end 127.75 62.75) (width 0.2) (layer "B.Cu") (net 12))
 (segment (start 136.75 69.25) (end 135 71) (width 0.2) (layer "F.Cu") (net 10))
 (segment (start 136.75 34.545) (end 136.75 69.25) (width 0.2) (layer "F.Cu") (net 10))
 (via (at 135 71) (size 0.6) (drill 0.3) (layers "F.Cu" "B.Cu") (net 10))
 (segment (start 135 71) (end 128.96 77.04) (width 0.2) (layer "B.Cu") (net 10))
 (segment (start 128.96 77.04) (end 128.96 79.25) (width 0.2) (layer "B.Cu") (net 10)))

